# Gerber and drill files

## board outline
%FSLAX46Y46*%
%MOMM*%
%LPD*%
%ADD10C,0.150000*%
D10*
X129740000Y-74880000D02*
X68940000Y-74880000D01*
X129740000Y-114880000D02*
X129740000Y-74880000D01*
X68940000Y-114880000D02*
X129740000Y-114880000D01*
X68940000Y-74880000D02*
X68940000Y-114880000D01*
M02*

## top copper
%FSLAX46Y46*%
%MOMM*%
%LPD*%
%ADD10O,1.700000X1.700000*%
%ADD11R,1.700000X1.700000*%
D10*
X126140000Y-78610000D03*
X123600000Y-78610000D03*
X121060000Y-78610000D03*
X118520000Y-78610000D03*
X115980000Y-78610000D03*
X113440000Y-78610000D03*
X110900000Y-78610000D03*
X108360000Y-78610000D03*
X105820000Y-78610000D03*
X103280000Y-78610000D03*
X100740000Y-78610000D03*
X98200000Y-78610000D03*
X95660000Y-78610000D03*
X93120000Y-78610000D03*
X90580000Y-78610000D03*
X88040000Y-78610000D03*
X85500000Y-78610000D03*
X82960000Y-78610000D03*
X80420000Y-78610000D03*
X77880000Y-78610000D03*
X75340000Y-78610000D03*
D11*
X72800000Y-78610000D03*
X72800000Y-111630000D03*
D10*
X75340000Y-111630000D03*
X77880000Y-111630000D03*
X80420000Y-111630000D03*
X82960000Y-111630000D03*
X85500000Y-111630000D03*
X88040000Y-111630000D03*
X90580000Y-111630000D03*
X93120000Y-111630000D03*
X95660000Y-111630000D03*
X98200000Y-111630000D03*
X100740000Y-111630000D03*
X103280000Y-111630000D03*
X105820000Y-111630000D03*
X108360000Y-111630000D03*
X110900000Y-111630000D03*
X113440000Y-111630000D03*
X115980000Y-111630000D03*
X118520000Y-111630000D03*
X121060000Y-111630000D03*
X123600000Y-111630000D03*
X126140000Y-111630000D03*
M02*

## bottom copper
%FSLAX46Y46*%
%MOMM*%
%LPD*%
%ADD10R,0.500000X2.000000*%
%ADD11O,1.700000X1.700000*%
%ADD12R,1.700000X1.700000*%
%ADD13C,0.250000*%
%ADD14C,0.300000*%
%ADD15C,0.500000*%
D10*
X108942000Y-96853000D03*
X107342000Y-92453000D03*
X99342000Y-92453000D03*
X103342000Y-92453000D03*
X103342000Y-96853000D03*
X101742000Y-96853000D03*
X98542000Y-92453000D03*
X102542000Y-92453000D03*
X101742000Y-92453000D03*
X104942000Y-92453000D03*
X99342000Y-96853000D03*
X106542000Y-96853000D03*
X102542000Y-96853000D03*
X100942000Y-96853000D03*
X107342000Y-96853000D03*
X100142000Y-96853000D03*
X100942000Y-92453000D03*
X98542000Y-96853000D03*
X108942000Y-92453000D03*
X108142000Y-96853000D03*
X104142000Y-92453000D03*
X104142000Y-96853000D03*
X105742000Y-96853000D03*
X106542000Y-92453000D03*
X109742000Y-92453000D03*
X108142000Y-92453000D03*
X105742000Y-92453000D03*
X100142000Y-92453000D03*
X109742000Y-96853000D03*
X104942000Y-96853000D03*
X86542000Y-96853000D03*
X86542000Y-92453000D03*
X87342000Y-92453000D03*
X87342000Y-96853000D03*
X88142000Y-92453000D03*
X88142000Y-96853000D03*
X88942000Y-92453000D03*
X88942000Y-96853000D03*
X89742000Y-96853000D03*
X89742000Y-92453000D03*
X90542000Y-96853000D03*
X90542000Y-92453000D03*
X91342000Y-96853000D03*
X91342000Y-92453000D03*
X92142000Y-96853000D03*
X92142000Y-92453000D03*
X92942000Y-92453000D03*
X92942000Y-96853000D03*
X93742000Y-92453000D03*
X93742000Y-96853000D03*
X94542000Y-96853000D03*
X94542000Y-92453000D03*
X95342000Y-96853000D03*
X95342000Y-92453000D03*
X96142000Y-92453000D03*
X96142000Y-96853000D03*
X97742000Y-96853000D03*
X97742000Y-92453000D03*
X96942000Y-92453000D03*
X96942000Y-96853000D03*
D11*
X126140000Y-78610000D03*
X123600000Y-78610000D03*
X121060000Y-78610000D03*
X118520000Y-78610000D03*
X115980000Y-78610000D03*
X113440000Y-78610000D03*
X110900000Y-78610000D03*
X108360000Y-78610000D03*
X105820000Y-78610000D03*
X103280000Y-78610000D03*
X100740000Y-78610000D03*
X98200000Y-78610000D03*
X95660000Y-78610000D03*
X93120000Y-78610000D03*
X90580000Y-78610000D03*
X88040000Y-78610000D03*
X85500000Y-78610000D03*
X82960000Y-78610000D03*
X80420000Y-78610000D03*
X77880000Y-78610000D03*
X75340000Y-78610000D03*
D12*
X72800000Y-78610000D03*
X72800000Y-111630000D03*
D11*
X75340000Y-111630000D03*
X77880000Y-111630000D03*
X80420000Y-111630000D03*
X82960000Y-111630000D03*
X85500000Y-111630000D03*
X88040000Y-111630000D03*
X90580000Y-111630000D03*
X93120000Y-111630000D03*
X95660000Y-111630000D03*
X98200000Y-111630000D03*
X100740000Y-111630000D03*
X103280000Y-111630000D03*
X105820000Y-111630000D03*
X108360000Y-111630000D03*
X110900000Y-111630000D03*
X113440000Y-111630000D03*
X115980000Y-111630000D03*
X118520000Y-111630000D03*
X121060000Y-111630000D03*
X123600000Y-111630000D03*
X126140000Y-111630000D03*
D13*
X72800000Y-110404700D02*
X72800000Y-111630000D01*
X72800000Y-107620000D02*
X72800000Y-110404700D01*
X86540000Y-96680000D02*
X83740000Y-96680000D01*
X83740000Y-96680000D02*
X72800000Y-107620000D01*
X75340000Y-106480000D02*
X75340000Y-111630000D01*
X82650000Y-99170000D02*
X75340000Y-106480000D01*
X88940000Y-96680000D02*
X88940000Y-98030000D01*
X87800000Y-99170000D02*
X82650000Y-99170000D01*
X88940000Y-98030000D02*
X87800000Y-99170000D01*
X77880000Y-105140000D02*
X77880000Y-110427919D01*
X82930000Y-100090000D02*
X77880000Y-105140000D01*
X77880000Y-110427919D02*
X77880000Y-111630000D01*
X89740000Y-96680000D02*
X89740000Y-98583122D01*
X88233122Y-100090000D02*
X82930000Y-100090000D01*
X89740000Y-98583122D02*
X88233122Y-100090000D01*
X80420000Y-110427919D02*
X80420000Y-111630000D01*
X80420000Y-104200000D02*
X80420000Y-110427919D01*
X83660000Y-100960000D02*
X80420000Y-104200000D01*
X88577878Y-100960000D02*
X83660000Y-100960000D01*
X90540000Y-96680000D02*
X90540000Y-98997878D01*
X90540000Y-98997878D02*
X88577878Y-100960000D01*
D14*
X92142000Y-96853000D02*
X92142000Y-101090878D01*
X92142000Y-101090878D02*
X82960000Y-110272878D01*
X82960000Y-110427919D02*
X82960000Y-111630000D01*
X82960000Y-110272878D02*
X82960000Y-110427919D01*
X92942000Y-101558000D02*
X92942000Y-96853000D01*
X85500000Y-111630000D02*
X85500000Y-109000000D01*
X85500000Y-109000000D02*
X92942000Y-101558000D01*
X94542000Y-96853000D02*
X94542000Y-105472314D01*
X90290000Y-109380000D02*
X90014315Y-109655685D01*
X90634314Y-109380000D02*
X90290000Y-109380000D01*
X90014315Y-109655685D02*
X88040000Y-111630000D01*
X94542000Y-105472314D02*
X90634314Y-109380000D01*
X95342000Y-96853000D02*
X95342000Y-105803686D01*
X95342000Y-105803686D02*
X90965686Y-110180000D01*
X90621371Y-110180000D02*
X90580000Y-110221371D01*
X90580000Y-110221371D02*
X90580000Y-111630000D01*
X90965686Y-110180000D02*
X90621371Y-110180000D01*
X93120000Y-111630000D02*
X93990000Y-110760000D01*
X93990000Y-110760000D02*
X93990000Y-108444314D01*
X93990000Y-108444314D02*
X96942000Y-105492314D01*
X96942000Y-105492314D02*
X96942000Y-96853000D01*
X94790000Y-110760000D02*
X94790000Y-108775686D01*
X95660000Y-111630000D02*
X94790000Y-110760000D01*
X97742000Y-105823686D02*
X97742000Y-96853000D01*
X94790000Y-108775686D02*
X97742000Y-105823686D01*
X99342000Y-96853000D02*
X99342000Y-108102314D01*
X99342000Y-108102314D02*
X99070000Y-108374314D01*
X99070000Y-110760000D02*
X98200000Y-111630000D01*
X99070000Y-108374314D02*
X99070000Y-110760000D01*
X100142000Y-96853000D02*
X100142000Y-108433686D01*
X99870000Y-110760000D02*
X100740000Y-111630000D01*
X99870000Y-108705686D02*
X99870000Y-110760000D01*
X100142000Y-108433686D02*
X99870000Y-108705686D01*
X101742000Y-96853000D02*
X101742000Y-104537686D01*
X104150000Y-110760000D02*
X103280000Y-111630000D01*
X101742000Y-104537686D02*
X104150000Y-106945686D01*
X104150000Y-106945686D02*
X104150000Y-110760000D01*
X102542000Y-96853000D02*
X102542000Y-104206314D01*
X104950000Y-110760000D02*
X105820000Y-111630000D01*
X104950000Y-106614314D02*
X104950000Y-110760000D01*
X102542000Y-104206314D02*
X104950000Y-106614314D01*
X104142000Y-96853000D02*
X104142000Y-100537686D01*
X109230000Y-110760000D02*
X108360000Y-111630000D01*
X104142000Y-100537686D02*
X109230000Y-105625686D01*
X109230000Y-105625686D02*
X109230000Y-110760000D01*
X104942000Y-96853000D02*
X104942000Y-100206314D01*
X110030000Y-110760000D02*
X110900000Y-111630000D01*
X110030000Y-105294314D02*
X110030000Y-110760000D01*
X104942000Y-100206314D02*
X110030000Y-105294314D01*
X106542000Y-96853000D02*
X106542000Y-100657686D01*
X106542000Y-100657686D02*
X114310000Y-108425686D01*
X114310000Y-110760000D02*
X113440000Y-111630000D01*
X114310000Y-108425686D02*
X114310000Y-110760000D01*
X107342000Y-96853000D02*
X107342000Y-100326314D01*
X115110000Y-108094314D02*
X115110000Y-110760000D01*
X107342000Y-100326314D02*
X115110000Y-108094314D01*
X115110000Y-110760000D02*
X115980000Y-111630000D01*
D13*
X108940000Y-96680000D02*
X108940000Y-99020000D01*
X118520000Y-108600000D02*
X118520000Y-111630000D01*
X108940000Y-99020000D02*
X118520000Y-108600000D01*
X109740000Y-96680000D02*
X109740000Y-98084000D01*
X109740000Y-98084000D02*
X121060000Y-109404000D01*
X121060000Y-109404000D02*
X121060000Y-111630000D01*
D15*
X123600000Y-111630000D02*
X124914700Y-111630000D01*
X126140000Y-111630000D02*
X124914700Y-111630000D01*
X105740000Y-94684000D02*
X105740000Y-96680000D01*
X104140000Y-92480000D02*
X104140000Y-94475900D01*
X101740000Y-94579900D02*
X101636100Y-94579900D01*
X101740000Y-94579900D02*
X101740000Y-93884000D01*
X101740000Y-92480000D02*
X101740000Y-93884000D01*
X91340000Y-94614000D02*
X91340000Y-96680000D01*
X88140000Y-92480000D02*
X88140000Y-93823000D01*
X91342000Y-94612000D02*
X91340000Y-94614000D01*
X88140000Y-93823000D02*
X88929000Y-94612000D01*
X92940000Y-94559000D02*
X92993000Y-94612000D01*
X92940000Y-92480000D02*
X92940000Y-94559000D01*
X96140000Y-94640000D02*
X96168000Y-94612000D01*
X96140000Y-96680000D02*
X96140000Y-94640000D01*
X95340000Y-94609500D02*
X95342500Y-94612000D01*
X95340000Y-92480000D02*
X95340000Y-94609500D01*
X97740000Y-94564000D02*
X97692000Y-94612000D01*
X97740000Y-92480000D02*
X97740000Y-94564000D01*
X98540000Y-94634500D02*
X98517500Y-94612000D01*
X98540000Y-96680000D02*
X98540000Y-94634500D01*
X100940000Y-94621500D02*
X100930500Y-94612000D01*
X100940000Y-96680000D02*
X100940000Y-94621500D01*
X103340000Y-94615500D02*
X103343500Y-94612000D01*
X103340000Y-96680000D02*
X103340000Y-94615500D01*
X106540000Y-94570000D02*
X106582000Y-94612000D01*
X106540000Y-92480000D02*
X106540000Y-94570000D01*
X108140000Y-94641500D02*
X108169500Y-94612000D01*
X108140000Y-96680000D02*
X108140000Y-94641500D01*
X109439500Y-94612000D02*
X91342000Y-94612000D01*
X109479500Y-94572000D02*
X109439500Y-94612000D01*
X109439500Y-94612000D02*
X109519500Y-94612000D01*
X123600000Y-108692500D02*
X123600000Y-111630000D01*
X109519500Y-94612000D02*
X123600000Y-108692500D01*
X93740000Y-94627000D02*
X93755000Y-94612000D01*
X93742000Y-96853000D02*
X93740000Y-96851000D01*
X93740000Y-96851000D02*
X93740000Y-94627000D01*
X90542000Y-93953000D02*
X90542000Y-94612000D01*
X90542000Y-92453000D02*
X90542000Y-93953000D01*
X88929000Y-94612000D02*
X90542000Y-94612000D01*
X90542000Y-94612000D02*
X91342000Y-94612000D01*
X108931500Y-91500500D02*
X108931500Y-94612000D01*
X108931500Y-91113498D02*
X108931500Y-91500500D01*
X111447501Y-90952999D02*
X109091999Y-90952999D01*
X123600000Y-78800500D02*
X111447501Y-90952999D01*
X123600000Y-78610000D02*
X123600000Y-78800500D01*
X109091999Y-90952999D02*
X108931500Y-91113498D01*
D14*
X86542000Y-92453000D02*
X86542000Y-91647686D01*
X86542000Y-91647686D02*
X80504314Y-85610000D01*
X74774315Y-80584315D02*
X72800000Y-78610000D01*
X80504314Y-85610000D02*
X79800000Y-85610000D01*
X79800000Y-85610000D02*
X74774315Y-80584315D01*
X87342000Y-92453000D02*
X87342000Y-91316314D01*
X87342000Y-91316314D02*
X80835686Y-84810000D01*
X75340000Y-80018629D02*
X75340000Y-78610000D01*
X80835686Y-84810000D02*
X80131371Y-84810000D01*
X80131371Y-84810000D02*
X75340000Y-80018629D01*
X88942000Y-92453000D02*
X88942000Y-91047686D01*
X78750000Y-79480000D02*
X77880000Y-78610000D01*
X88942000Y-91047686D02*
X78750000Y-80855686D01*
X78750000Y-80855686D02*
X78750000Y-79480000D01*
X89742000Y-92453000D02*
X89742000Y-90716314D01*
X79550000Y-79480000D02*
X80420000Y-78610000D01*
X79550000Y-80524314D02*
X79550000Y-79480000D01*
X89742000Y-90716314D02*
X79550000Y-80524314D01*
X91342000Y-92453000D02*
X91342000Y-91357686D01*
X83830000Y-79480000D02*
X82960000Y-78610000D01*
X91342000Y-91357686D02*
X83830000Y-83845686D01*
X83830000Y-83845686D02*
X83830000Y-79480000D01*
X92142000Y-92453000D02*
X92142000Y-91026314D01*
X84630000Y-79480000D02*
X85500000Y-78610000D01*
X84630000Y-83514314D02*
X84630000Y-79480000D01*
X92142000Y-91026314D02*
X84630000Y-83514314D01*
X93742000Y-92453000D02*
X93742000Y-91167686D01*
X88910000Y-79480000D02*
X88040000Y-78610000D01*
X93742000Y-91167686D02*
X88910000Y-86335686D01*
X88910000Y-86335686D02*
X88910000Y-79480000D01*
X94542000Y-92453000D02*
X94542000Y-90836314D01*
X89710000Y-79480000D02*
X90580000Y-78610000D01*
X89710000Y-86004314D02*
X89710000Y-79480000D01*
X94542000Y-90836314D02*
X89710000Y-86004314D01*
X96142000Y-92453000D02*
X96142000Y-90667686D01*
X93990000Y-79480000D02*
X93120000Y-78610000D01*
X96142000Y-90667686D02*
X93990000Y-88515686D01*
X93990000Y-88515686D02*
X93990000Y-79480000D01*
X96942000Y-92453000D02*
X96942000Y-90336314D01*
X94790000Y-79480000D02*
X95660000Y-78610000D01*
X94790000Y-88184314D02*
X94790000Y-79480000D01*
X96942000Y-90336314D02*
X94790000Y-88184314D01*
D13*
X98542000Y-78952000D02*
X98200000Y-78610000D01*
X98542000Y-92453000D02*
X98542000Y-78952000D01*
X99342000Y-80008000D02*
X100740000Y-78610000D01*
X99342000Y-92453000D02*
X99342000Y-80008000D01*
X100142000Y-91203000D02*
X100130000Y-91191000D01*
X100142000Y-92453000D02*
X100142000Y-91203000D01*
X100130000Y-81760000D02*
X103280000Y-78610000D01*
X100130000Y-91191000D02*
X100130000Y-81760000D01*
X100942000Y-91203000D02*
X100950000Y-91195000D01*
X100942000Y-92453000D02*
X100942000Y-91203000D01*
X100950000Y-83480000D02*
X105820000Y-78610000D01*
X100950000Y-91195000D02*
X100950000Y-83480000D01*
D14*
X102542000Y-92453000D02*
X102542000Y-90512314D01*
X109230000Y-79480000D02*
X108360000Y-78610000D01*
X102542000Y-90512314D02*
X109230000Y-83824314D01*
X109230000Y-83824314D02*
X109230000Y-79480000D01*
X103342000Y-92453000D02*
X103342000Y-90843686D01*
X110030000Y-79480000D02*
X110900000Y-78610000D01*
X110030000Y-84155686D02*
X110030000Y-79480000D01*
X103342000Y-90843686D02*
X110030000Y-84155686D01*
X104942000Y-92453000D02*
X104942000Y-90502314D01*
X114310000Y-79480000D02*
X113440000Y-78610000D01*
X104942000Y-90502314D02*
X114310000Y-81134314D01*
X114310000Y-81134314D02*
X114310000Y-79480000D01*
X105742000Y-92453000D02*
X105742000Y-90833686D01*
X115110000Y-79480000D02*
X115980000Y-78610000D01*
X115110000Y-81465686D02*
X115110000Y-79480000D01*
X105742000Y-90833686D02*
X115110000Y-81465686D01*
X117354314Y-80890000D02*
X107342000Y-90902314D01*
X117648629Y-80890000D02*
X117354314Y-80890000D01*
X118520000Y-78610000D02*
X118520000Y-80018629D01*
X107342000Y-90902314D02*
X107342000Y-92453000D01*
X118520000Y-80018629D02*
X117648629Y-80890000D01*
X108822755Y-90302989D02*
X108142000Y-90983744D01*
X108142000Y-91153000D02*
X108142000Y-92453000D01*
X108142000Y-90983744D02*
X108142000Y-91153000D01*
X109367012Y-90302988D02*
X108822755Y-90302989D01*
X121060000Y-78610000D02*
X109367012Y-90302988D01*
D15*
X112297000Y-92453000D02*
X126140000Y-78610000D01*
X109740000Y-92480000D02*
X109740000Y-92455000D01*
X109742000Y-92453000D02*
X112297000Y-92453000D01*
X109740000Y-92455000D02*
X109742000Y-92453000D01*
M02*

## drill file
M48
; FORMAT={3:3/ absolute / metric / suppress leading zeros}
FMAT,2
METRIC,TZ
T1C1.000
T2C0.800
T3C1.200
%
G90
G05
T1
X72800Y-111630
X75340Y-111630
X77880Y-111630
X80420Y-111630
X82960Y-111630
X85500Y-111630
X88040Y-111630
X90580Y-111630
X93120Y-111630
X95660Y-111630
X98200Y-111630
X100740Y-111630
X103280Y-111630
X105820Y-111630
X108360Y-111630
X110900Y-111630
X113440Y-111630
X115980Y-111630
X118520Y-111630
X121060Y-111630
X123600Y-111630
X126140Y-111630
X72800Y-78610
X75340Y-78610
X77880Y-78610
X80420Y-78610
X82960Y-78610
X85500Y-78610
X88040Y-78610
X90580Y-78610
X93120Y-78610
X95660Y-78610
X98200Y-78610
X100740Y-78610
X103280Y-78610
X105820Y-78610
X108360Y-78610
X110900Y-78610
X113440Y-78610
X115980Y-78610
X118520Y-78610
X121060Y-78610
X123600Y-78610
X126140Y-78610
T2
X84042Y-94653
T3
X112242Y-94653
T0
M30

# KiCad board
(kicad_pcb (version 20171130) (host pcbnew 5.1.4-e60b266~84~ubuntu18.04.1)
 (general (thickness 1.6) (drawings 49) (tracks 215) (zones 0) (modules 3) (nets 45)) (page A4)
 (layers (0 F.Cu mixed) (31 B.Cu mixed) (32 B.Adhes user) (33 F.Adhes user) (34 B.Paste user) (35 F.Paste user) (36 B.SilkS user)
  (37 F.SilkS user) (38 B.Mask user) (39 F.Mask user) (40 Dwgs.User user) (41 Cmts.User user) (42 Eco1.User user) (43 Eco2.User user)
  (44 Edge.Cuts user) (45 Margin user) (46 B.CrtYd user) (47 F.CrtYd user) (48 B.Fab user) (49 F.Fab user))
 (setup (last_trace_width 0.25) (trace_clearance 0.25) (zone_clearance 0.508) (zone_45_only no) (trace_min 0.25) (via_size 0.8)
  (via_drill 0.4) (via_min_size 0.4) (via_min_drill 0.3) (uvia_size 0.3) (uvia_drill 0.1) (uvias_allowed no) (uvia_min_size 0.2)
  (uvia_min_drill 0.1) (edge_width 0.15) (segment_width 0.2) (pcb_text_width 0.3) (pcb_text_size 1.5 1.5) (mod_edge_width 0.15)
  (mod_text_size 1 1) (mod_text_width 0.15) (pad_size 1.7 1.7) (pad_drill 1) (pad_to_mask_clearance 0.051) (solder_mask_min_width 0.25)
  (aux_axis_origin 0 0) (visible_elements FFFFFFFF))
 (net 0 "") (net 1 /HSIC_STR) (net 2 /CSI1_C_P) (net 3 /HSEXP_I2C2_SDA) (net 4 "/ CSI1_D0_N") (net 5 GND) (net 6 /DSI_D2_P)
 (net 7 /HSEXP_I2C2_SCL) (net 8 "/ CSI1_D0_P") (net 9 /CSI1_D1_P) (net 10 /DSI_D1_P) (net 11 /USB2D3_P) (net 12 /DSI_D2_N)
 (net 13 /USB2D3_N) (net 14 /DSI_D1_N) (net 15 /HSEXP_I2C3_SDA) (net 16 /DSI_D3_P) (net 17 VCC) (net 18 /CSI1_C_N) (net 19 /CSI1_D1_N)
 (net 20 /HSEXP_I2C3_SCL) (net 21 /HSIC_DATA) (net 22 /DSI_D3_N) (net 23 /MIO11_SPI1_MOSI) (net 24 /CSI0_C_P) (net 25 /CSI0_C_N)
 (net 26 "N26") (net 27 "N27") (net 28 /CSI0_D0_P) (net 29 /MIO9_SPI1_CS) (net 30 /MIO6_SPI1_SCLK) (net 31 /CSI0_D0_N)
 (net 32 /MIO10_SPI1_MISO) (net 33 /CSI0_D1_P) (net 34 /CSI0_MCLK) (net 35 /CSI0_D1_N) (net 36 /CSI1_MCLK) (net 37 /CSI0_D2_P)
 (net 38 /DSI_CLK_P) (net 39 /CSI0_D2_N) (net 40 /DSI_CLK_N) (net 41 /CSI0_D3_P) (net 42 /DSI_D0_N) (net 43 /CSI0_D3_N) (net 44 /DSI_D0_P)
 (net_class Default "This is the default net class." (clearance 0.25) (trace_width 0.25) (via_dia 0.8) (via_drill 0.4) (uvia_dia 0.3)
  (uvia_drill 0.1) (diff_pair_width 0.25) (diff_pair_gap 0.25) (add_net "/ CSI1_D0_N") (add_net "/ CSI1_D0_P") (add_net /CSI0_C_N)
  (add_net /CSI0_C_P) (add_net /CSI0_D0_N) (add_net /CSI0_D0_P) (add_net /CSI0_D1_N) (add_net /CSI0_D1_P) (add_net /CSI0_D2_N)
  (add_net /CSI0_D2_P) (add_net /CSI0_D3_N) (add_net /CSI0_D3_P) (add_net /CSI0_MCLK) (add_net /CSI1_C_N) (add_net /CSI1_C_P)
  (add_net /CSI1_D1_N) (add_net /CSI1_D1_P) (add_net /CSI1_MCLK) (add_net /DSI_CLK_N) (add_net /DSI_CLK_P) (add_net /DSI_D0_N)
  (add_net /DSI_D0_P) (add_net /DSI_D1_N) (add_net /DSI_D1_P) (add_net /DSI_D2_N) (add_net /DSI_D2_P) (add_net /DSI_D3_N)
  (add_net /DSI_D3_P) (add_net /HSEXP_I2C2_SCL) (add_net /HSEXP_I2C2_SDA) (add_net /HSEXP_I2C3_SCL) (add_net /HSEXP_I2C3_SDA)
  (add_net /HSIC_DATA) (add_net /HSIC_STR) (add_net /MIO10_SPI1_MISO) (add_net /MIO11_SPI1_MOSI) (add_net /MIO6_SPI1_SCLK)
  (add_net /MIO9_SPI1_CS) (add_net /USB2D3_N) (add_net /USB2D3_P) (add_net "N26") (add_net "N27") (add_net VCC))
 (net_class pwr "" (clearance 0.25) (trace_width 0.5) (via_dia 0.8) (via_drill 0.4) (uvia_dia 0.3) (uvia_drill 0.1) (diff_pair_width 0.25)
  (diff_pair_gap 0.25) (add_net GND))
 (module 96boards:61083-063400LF (layer B.Cu) (at 98.142 94.653)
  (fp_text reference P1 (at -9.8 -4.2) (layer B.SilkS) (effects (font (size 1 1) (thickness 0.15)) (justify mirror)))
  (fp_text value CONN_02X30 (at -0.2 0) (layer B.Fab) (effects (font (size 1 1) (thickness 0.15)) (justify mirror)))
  (pad 57 smd rect (at 10.8 2.2) (size 0.5 2) (layers B.Cu B.Paste B.Mask) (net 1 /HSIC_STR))
  (pad 54 smd rect (at 9.2 -2.2) (size 0.5 2) (layers B.Cu B.Paste B.Mask) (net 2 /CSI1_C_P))
  (pad 34 smd rect (at 1.2 -2.2) (size 0.5 2) (layers B.Cu B.Paste B.Mask) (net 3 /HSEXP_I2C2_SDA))
  (pad 44 smd rect (at 5.2 -2.2) (size 0.5 2) (layers B.Cu B.Paste B.Mask) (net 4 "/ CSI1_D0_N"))
  (pad 43 smd rect (at 5.2 2.2) (size 0.5 2) (layers B.Cu B.Paste B.Mask) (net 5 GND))
  (pad 39 smd rect (at 3.6 2.2) (size 0.5 2) (layers B.Cu B.Paste B.Mask) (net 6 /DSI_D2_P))
  (pad 32 smd rect (at 0.4 -2.2) (size 0.5 2) (layers B.Cu B.Paste B.Mask) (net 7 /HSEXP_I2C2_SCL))
  (pad 42 smd rect (at 4.4 -2.2) (size 0.5 2) (layers B.Cu B.Paste B.Mask) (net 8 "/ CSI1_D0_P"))
  (pad 40 smd rect (at 3.6 -2.2) (size 0.5 2) (layers B.Cu B.Paste B.Mask) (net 5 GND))
  (pad 48 smd rect (at 6.8 -2.2) (size 0.5 2) (layers B.Cu B.Paste B.Mask) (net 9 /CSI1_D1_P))
  (pad 33 smd rect (at 1.2 2.2) (size 0.5 2) (layers B.Cu B.Paste B.Mask) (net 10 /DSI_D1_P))
  (pad 51 smd rect (at 8.4 2.2) (size 0.5 2) (layers B.Cu B.Paste B.Mask) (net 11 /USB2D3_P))
  (pad 41 smd rect (at 4.4 2.2) (size 0.5 2) (layers B.Cu B.Paste B.Mask) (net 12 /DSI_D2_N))
  (pad 37 smd rect (at 2.8 2.2) (size 0.5 2) (layers B.Cu B.Paste B.Mask) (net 5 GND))
  (pad 53 smd rect (at 9.2 2.2) (size 0.5 2) (layers B.Cu B.Paste B.Mask) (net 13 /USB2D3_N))
  (pad 35 smd rect (at 2 2.2) (size 0.5 2) (layers B.Cu B.Paste B.Mask) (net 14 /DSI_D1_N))
  (pad 38 smd rect (at 2.8 -2.2) (size 0.5 2) (layers B.Cu B.Paste B.Mask) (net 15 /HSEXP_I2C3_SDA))
  (pad 31 smd rect (at 0.4 2.2) (size 0.5 2) (layers B.Cu B.Paste B.Mask) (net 5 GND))
  (pad 58 smd rect (at 10.8 -2.2) (size 0.5 2) (layers B.Cu B.Paste B.Mask) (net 5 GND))
  (pad 55 smd rect (at 10 2.2) (size 0.5 2) (layers B.Cu B.Paste B.Mask) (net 5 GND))
  (pad 46 smd rect (at 6 -2.2) (size 0.5 2) (layers B.Cu B.Paste B.Mask) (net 5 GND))
  (pad 45 smd rect (at 6 2.2) (size 0.5 2) (layers B.Cu B.Paste B.Mask) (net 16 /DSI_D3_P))
  (pad 49 smd rect (at 7.6 2.2) (size 0.5 2) (layers B.Cu B.Paste B.Mask) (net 5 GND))
  (pad 52 smd rect (at 8.4 -2.2) (size 0.5 2) (layers B.Cu B.Paste B.Mask) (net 5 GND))
  (pad 60 smd rect (at 11.6 -2.2) (size 0.5 2) (layers B.Cu B.Paste B.Mask) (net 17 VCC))
  (pad 56 smd rect (at 10 -2.2) (size 0.5 2) (layers B.Cu B.Paste B.Mask) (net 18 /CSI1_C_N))
  (pad 50 smd rect (at 7.6 -2.2) (size 0.5 2) (layers B.Cu B.Paste B.Mask) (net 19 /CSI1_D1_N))
  (pad 36 smd rect (at 2 -2.2) (size 0.5 2) (layers B.Cu B.Paste B.Mask) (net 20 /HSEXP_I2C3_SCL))
  (pad 59 smd rect (at 11.6 2.2) (size 0.5 2) (layers B.Cu B.Paste B.Mask) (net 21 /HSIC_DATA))
  (pad 47 smd rect (at 6.8 2.2) (size 0.5 2) (layers B.Cu B.Paste B.Mask) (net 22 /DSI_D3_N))
  (pad "" np_thru_hole circle (at 14.1 0) (size 1.2 1.2) (drill 1.2) (layers *.Cu *.Mask))
  (pad 1 smd rect (at -11.6 2.2) (size 0.5 2) (layers B.Cu B.Paste B.Mask) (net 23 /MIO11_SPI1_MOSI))
  (pad 2 smd rect (at -11.6 -2.2) (size 0.5 2) (layers B.Cu B.Paste B.Mask) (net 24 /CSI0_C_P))
  (pad 4 smd rect (at -10.8 -2.2) (size 0.5 2) (layers B.Cu B.Paste B.Mask) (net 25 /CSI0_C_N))
  (pad 3 smd rect (at -10.8 2.2) (size 0.5 2) (layers B.Cu B.Paste B.Mask) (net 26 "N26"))
  (pad 6 smd rect (at -10 -2.2) (size 0.5 2) (layers B.Cu B.Paste B.Mask) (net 5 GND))
  (pad 5 smd rect (at -10 2.2) (size 0.5 2) (layers B.Cu B.Paste B.Mask) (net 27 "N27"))
  (pad 8 smd rect (at -9.2 -2.2) (size 0.5 2) (layers B.Cu B.Paste B.Mask) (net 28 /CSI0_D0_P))
  (pad 7 smd rect (at -9.2 2.2) (size 0.5 2) (layers B.Cu B.Paste B.Mask) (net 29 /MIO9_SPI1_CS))
  (pad 9 smd rect (at -8.4 2.2) (size 0.5 2) (layers B.Cu B.Paste B.Mask) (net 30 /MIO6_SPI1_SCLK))
  (pad 10 smd rect (at -8.4 -2.2) (size 0.5 2) (layers B.Cu B.Paste B.Mask) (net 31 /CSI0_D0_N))
  (pad 11 smd rect (at -7.6 2.2) (size 0.5 2) (layers B.Cu B.Paste B.Mask) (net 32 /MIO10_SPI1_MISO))
  (pad 12 smd rect (at -7.6 -2.2) (size 0.5 2) (layers B.Cu B.Paste B.Mask) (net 5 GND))
  (pad 13 smd rect (at -6.8 2.2) (size 0.5 2) (layers B.Cu B.Paste B.Mask) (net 5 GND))
  (pad 14 smd rect (at -6.8 -2.2) (size 0.5 2) (layers B.Cu B.Paste B.Mask) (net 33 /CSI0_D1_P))
  (pad 15 smd rect (at -6 2.2) (size 0.5 2) (layers B.Cu B.Paste B.Mask) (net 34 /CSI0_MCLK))
  (pad 16 smd rect (at -6 -2.2) (size 0.5 2) (layers B.Cu B.Paste B.Mask) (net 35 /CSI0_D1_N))
  (pad 18 smd rect (at -5.2 -2.2) (size 0.5 2) (layers B.Cu B.Paste B.Mask) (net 5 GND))
  (pad 17 smd rect (at -5.2 2.2) (size 0.5 2) (layers B.Cu B.Paste B.Mask) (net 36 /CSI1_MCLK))
  (pad 20 smd rect (at -4.4 -2.2) (size 0.5 2) (layers B.Cu B.Paste B.Mask) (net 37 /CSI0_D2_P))
  (pad 19 smd rect (at -4.4 2.2) (size 0.5 2) (layers B.Cu B.Paste B.Mask) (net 5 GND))
  (pad 21 smd rect (at -3.6 2.2) (size 0.5 2) (layers B.Cu B.Paste B.Mask) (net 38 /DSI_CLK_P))
  (pad 22 smd rect (at -3.6 -2.2) (size 0.5 2) (layers B.Cu B.Paste B.Mask) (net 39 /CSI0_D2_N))
  (pad 23 smd rect (at -2.8 2.2) (size 0.5 2) (layers B.Cu B.Paste B.Mask) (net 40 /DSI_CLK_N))
  (pad 24 smd rect (at -2.8 -2.2) (size 0.5 2) (layers B.Cu B.Paste B.Mask) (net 5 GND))
  (pad 26 smd rect (at -2 -2.2) (size 0.5 2) (layers B.Cu B.Paste B.Mask) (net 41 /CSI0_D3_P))
  (pad 25 smd rect (at -2 2.2) (size 0.5 2) (layers B.Cu B.Paste B.Mask) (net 5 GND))
  (pad 29 smd rect (at -0.4 2.2) (size 0.5 2) (layers B.Cu B.Paste B.Mask) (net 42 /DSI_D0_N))
  (pad 30 smd rect (at -0.4 -2.2) (size 0.5 2) (layers B.Cu B.Paste B.Mask) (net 5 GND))
  (pad 28 smd rect (at -1.2 -2.2) (size 0.5 2) (layers B.Cu B.Paste B.Mask) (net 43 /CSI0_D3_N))
  (pad 27 smd rect (at -1.2 2.2) (size 0.5 2) (layers B.Cu B.Paste B.Mask) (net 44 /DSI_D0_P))
  (pad "" np_thru_hole circle (at -14.1 0) (size 0.8 0.8) (drill 0.8) (layers *.Cu *.Mask)))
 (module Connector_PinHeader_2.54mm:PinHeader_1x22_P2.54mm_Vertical (layer F.Cu) (at 72.8 78.61 90)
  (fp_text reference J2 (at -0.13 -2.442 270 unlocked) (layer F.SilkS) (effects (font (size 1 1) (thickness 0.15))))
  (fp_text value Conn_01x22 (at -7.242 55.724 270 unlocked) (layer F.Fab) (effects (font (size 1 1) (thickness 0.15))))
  (pad 22 thru_hole oval (at 0 53.34 90) (size 1.7 1.7) (drill 1) (layers *.Cu *.Mask) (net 17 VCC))
  (pad 21 thru_hole oval (at 0 50.8 90) (size 1.7 1.7) (drill 1) (layers *.Cu *.Mask) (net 5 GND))
  (pad 20 thru_hole oval (at 0 48.26 90) (size 1.7 1.7) (drill 1) (layers *.Cu *.Mask) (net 18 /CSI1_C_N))
  (pad 19 thru_hole oval (at 0 45.72 90) (size 1.7 1.7) (drill 1) (layers *.Cu *.Mask) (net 2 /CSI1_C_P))
  (pad 18 thru_hole oval (at 0 43.18 90) (size 1.7 1.7) (drill 1) (layers *.Cu *.Mask) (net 19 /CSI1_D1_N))
  (pad 17 thru_hole oval (at 0 40.64 90) (size 1.7 1.7) (drill 1) (layers *.Cu *.Mask) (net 9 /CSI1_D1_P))
  (pad 16 thru_hole oval (at 0 38.1 90) (size 1.7 1.7) (drill 1) (layers *.Cu *.Mask) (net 4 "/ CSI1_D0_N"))
  (pad 15 thru_hole oval (at 0 35.56 90) (size 1.7 1.7) (drill 1) (layers *.Cu *.Mask) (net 8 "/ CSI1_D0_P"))
  (pad 14 thru_hole oval (at 0 33.02 90) (size 1.7 1.7) (drill 1) (layers *.Cu *.Mask) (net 15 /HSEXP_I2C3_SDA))
  (pad 13 thru_hole oval (at 0 30.48 90) (size 1.7 1.7) (drill 1) (layers *.Cu *.Mask) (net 20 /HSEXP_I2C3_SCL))
  (pad 12 thru_hole oval (at 0 27.94 90) (size 1.7 1.7) (drill 1) (layers *.Cu *.Mask) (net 3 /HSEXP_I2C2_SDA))
  (pad 11 thru_hole oval (at 0 25.4 90) (size 1.7 1.7) (drill 1) (layers *.Cu *.Mask) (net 7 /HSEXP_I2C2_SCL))
  (pad 10 thru_hole oval (at 0 22.86 90) (size 1.7 1.7) (drill 1) (layers *.Cu *.Mask) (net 43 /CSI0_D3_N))
  (pad 9 thru_hole oval (at 0 20.32 90) (size 1.7 1.7) (drill 1) (layers *.Cu *.Mask) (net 41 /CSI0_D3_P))
  (pad 8 thru_hole oval (at 0 17.78 90) (size 1.7 1.7) (drill 1) (layers *.Cu *.Mask) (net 39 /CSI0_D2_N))
  (pad 7 thru_hole oval (at 0 15.24 90) (size 1.7 1.7) (drill 1) (layers *.Cu *.Mask) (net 37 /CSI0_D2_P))
  (pad 6 thru_hole oval (at 0 12.7 90) (size 1.7 1.7) (drill 1) (layers *.Cu *.Mask) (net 35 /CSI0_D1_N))
  (pad 5 thru_hole oval (at 0 10.16 90) (size 1.7 1.7) (drill 1) (layers *.Cu *.Mask) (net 33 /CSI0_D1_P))
  (pad 4 thru_hole oval (at 0 7.62 90) (size 1.7 1.7) (drill 1) (layers *.Cu *.Mask) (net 31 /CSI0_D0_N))
  (pad 3 thru_hole oval (at 0 5.08 90) (size 1.7 1.7) (drill 1) (layers *.Cu *.Mask) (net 28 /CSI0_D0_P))
  (pad 2 thru_hole oval (at 0 2.54 90) (size 1.7 1.7) (drill 1) (layers *.Cu *.Mask) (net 25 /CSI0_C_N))
  (pad 1 thru_hole rect (at 0 0 90) (size 1.7 1.7) (drill 1) (layers *.Cu *.Mask) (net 24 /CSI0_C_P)))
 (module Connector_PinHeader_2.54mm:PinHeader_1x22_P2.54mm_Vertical (layer F.Cu) (at 72.8 111.63 90)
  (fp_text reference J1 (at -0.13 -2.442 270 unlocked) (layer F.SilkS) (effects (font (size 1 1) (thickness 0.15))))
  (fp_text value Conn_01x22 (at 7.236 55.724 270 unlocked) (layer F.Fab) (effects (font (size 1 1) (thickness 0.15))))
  (pad 1 thru_hole rect (at 0 0 90) (size 1.7 1.7) (drill 1) (layers *.Cu *.SilkS *.Mask) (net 23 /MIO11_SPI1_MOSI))
  (pad 2 thru_hole oval (at 0 2.54 90) (size 1.7 1.7) (drill 1) (layers *.Cu *.Mask) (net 29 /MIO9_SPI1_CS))
  (pad 3 thru_hole oval (at 0 5.08 90) (size 1.7 1.7) (drill 1) (layers *.Cu *.Mask) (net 30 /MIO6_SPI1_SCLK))
  (pad 4 thru_hole oval (at 0 7.62 90) (size 1.7 1.7) (drill 1) (layers *.Cu *.Mask) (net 32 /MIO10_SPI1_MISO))
  (pad 5 thru_hole oval (at 0 10.16 90) (size 1.7 1.7) (drill 1) (layers *.Cu *.Mask) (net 34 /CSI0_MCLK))
  (pad 6 thru_hole oval (at 0 12.7 90) (size 1.7 1.7) (drill 1) (layers *.Cu *.Mask) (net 36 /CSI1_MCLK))
  (pad 7 thru_hole oval (at 0 15.24 90) (size 1.7 1.7) (drill 1) (layers *.Cu *.Mask) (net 38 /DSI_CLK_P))
  (pad 8 thru_hole oval (at 0 17.78 90) (size 1.7 1.7) (drill 1) (layers *.Cu *.Mask) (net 40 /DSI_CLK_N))
  (pad 9 thru_hole oval (at 0 20.32 90) (size 1.7 1.7) (drill 1) (layers *.Cu *.Mask) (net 44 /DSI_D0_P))
  (pad 10 thru_hole oval (at 0 22.86 90) (size 1.7 1.7) (drill 1) (layers *.Cu *.Mask) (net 42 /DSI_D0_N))
  (pad 11 thru_hole oval (at 0 25.4 90) (size 1.7 1.7) (drill 1) (layers *.Cu *.Mask) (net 10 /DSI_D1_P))
  (pad 12 thru_hole oval (at 0 27.94 90) (size 1.7 1.7) (drill 1) (layers *.Cu *.Mask) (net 14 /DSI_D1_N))
  (pad 13 thru_hole oval (at 0 30.48 90) (size 1.7 1.7) (drill 1) (layers *.Cu *.Mask) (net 6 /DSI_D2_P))
  (pad 14 thru_hole oval (at 0 33.02 90) (size 1.7 1.7) (drill 1) (layers *.Cu *.Mask) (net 12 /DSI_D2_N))
  (pad 15 thru_hole oval (at 0 35.56 90) (size 1.7 1.7) (drill 1) (layers *.Cu *.Mask) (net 16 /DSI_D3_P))
  (pad 16 thru_hole oval (at 0 38.1 90) (size 1.7 1.7) (drill 1) (layers *.Cu *.Mask) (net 22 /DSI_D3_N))
  (pad 17 thru_hole oval (at 0 40.64 90) (size 1.7 1.7) (drill 1) (layers *.Cu *.Mask) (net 11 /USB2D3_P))
  (pad 18 thru_hole oval (at 0 43.18 90) (size 1.7 1.7) (drill 1) (layers *.Cu *.Mask) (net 13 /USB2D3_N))
  (pad 19 thru_hole oval (at 0 45.72 90) (size 1.7 1.7) (drill 1) (layers *.Cu *.Mask) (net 1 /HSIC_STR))
  (pad 20 thru_hole oval (at 0 48.26 90) (size 1.7 1.7) (drill 1) (layers *.Cu *.Mask) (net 21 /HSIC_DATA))
  (pad 21 thru_hole oval (at 0 50.8 90) (size 1.7 1.7) (drill 1) (layers *.Cu *.Mask) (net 5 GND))
  (pad 22 thru_hole oval (at 0 53.34 90) (size 1.7 1.7) (drill 1) (layers *.Cu *.Mask) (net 5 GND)))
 (gr_line (start 129.74 74.88) (end 68.94 74.88) (layer Edge.Cuts) (width 0.15))
 (gr_line (start 129.74 114.88) (end 129.74 74.88) (layer Edge.Cuts) (width 0.15))
 (gr_line (start 68.94 114.88) (end 129.74 114.88) (layer Edge.Cuts) (width 0.15))
 (gr_line (start 68.94 74.88) (end 68.94 114.88) (layer Edge.Cuts) (width 0.15))
 (segment (start 72.8 110.4047) (end 72.8 111.63) (width 0.25) (layer B.Cu) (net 23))
 (segment (start 72.8 107.62) (end 72.8 110.4047) (width 0.25) (layer B.Cu) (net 23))
 (segment (start 86.54 96.68) (end 83.74 96.68) (width 0.25) (layer B.Cu) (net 23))
 (segment (start 83.74 96.68) (end 72.8 107.62) (width 0.25) (layer B.Cu) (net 23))
 (segment (start 75.34 106.48) (end 75.34 111.63) (width 0.25) (layer B.Cu) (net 29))
 (segment (start 82.65 99.17) (end 75.34 106.48) (width 0.25) (layer B.Cu) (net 29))
 (segment (start 88.94 96.68) (end 88.94 98.03) (width 0.25) (layer B.Cu) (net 29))
 (segment (start 87.8 99.17) (end 82.65 99.17) (width 0.25) (layer B.Cu) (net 29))
 (segment (start 88.94 98.03) (end 87.8 99.17) (width 0.25) (layer B.Cu) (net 29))
 (segment (start 77.88 105.14) (end 77.88 110.427919) (width 0.25) (layer B.Cu) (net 30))
 (segment (start 82.93 100.09) (end 77.88 105.14) (width 0.25) (layer B.Cu) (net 30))
 (segment (start 77.88 110.427919) (end 77.88 111.63) (width 0.25) (layer B.Cu) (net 30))
 (segment (start 89.74 96.68) (end 89.74 98.583122) (width 0.25) (layer B.Cu) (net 30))
 (segment (start 88.233122 100.09) (end 82.93 100.09) (width 0.25) (layer B.Cu) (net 30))
 (segment (start 89.74 98.583122) (end 88.233122 100.09) (width 0.25) (layer B.Cu) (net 30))
 (segment (start 80.42 110.427919) (end 80.42 111.63) (width 0.25) (layer B.Cu) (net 32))
 (segment (start 80.42 104.2) (end 80.42 110.427919) (width 0.25) (layer B.Cu) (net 32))
 (segment (start 83.66 100.96) (end 80.42 104.2) (width 0.25) (layer B.Cu) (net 32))
 (segment (start 88.577878 100.96) (end 83.66 100.96) (width 0.25) (layer B.Cu) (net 32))
 (segment (start 90.54 96.68) (end 90.54 98.997878) (width 0.25) (layer B.Cu) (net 32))
 (segment (start 90.54 98.997878) (end 88.577878 100.96) (width 0.25) (layer B.Cu) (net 32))
 (segment (start 92.142 96.853) (end 92.142 101.090878) (width 0.3) (layer B.Cu) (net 34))
 (segment (start 92.142 101.090878) (end 82.96 110.272878) (width 0.3) (layer B.Cu) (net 34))
 (segment (start 82.96 110.427919) (end 82.96 111.63) (width 0.3) (layer B.Cu) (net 34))
 (segment (start 82.96 110.272878) (end 82.96 110.427919) (width 0.3) (layer B.Cu) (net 34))
 (segment (start 92.942 101.558) (end 92.942 96.853) (width 0.3) (layer B.Cu) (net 36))
 (segment (start 85.5 111.63) (end 85.5 109) (width 0.3) (layer B.Cu) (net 36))
 (segment (start 85.5 109) (end 92.942 101.558) (width 0.3) (layer B.Cu) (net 36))
 (segment (start 94.542 96.853) (end 94.542 105.472314) (width 0.3) (layer B.Cu) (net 38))
 (segment (start 90.29 109.38) (end 90.014315 109.655685) (width 0.3) (layer B.Cu) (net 38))
 (segment (start 90.634314 109.38) (end 90.29 109.38) (width 0.3) (layer B.Cu) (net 38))
 (segment (start 90.014315 109.655685) (end 88.04 111.63) (width 0.3) (layer B.Cu) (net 38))
 (segment (start 94.542 105.472314) (end 90.634314 109.38) (width 0.3) (layer B.Cu) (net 38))
 (segment (start 95.342 96.853) (end 95.342 105.803686) (width 0.3) (layer B.Cu) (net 40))
 (segment (start 95.342 105.803686) (end 90.965686 110.18) (width 0.3) (layer B.Cu) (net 40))
 (segment (start 90.621371 110.18) (end 90.58 110.221371) (width 0.3) (layer B.Cu) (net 40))
 (segment (start 90.58 110.221371) (end 90.58 111.63) (width 0.3) (layer B.Cu) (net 40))
 (segment (start 90.965686 110.18) (end 90.621371 110.18) (width 0.3) (layer B.Cu) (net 40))
 (segment (start 93.12 111.63) (end 93.99 110.76) (width 0.3) (layer B.Cu) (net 44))
 (segment (start 93.99 110.76) (end 93.99 108.444314) (width 0.3) (layer B.Cu) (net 44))
 (segment (start 93.99 108.444314) (end 96.942 105.492314) (width 0.3) (layer B.Cu) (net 44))
 (segment (start 96.942 105.492314) (end 96.942 96.853) (width 0.3) (layer B.Cu) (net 44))
 (segment (start 94.79 110.76) (end 94.79 108.775686) (width 0.3) (layer B.Cu) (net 42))
 (segment (start 95.66 111.63) (end 94.79 110.76) (width 0.3) (layer B.Cu) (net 42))
 (segment (start 97.742 105.823686) (end 97.742 96.853) (width 0.3) (layer B.Cu) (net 42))
 (segment (start 94.79 108.775686) (end 97.742 105.823686) (width 0.3) (layer B.Cu) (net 42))
 (segment (start 99.342 96.853) (end 99.342 108.102314) (width 0.3) (layer B.Cu) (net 10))
 (segment (start 99.342 108.102314) (end 99.07 108.374314) (width 0.3) (layer B.Cu) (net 10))
 (segment (start 99.07 110.76) (end 98.2 111.63) (width 0.3) (layer B.Cu) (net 10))
 (segment (start 99.07 108.374314) (end 99.07 110.76) (width 0.3) (layer B.Cu) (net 10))
 (segment (start 100.142 96.853) (end 100.142 108.433686) (width 0.3) (layer B.Cu) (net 14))
 (segment (start 99.87 110.76) (end 100.74 111.63) (width 0.3) (layer B.Cu) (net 14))
 (segment (start 99.87 108.705686) (end 99.87 110.76) (width 0.3) (layer B.Cu) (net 14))
 (segment (start 100.142 108.433686) (end 99.87 108.705686) (width 0.3) (layer B.Cu) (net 14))
 (segment (start 101.742 96.853) (end 101.742 104.537686) (width 0.3) (layer B.Cu) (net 6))
 (segment (start 104.15 110.76) (end 103.28 111.63) (width 0.3) (layer B.Cu) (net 6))
 (segment (start 101.742 104.537686) (end 104.15 106.945686) (width 0.3) (layer B.Cu) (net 6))
 (segment (start 104.15 106.945686) (end 104.15 110.76) (width 0.3) (layer B.Cu) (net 6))
 (segment (start 102.542 96.853) (end 102.542 104.206314) (width 0.3) (layer B.Cu) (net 12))
 (segment (start 104.95 110.76) (end 105.82 111.63) (width 0.3) (layer B.Cu) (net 12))
 (segment (start 104.95 106.614314) (end 104.95 110.76) (width 0.3) (layer B.Cu) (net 12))
 (segment (start 102.542 104.206314) (end 104.95 106.614314) (width 0.3) (layer B.Cu) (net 12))
 (segment (start 104.142 96.853) (end 104.142 100.537686) (width 0.3) (layer B.Cu) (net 16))
 (segment (start 109.23 110.76) (end 108.36 111.63) (width 0.3) (layer B.Cu) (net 16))
 (segment (start 104.142 100.537686) (end 109.23 105.625686) (width 0.3) (layer B.Cu) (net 16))
 (segment (start 109.23 105.625686) (end 109.23 110.76) (width 0.3) (layer B.Cu) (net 16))
 (segment (start 104.942 96.853) (end 104.942 100.206314) (width 0.3) (layer B.Cu) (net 22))
 (segment (start 110.03 110.76) (end 110.9 111.63) (width 0.3) (layer B.Cu) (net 22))
 (segment (start 110.03 105.294314) (end 110.03 110.76) (width 0.3) (layer B.Cu) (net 22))
 (segment (start 104.942 100.206314) (end 110.03 105.294314) (width 0.3) (layer B.Cu) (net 22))
 (segment (start 106.542 96.853) (end 106.542 100.657686) (width 0.3) (layer B.Cu) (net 11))
 (segment (start 106.542 100.657686) (end 114.31 108.425686) (width 0.3) (layer B.Cu) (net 11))
 (segment (start 114.31 110.76) (end 113.44 111.63) (width 0.3) (layer B.Cu) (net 11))
 (segment (start 114.31 108.425686) (end 114.31 110.76) (width 0.3) (layer B.Cu) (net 11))
 (segment (start 107.342 96.853) (end 107.342 100.326314) (width 0.3) (layer B.Cu) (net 13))
 (segment (start 115.11 108.094314) (end 115.11 110.76) (width 0.3) (layer B.Cu) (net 13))
 (segment (start 107.342 100.326314) (end 115.11 108.094314) (width 0.3) (layer B.Cu) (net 13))
 (segment (start 115.11 110.76) (end 115.98 111.63) (width 0.3) (layer B.Cu) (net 13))
 (segment (start 108.94 96.68) (end 108.94 99.02) (width 0.25) (layer B.Cu) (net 1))
 (segment (start 118.52 108.6) (end 118.52 111.63) (width 0.25) (layer B.Cu) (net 1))
 (segment (start 108.94 99.02) (end 118.52 108.6) (width 0.25) (layer B.Cu) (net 1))
 (segment (start 109.74 96.68) (end 109.74 98.084) (width 0.25) (layer B.Cu) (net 21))
 (segment (start 109.74 98.084) (end 121.06 109.404) (width 0.25) (layer B.Cu) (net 21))
 (segment (start 121.06 109.404) (end 121.06 111.63) (width 0.25) (layer B.Cu) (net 21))
 (segment (start 123.6 111.63) (end 124.9147 111.63) (width 0.5) (layer B.Cu) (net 5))
 (segment (start 126.14 111.63) (end 124.9147 111.63) (width 0.5) (layer B.Cu) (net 5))
 (segment (start 105.74 94.684) (end 105.74 96.68) (width 0.5) (layer B.Cu) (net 5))
 (segment (start 104.14 92.48) (end 104.14 94.4759) (width 0.5) (layer B.Cu) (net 5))
 (segment (start 101.74 94.5799) (end 101.6361 94.5799) (width 0.5) (layer B.Cu) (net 5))
 (segment (start 101.74 94.5799) (end 101.74 93.884) (width 0.5) (layer B.Cu) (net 5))
 (segment (start 101.74 92.48) (end 101.74 93.884) (width 0.5) (layer B.Cu) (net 5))
 (segment (start 91.34 94.614) (end 91.34 96.68) (width 0.5) (layer B.Cu) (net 5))
 (segment (start 88.14 92.48) (end 88.14 93.823) (width 0.5) (layer B.Cu) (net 5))
 (segment (start 91.342 94.612) (end 91.34 94.614) (width 0.5) (layer B.Cu) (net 5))
 (segment (start 88.14 93.823) (end 88.929 94.612) (width 0.5) (layer B.Cu) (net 5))
 (segment (start 92.94 94.559) (end 92.993 94.612) (width 0.5) (layer B.Cu) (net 5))
 (segment (start 92.94 92.48) (end 92.94 94.559) (width 0.5) (layer B.Cu) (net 5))
 (segment (start 96.14 94.64) (end 96.168 94.612) (width 0.5) (layer B.Cu) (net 5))
 (segment (start 96.14 96.68) (end 96.14 94.64) (width 0.5) (layer B.Cu) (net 5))
 (segment (start 95.34 94.6095) (end 95.3425 94.612) (width 0.5) (layer B.Cu) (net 5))
 (segment (start 95.34 92.48) (end 95.34 94.6095) (width 0.5) (layer B.Cu) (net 5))
 (segment (start 97.74 94.564) (end 97.692 94.612) (width 0.5) (layer B.Cu) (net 5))
 (segment (start 97.74 92.48) (end 97.74 94.564) (width 0.5) (layer B.Cu) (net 5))
 (segment (start 98.54 94.6345) (end 98.5175 94.612) (width 0.5) (layer B.Cu) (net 5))
 (segment (start 98.54 96.68) (end 98.54 94.6345) (width 0.5) (layer B.Cu) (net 5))
 (segment (start 100.94 94.6215) (end 100.9305 94.612) (width 0.5) (layer B.Cu) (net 5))
 (segment (start 100.94 96.68) (end 100.94 94.6215) (width 0.5) (layer B.Cu) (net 5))
 (segment (start 103.34 94.6155) (end 103.3435 94.612) (width 0.5) (layer B.Cu) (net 5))
 (segment (start 103.34 96.68) (end 103.34 94.6155) (width 0.5) (layer B.Cu) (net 5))
 (segment (start 106.54 94.57) (end 106.582 94.612) (width 0.5) (layer B.Cu) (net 5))
 (segment (start 106.54 92.48) (end 106.54 94.57) (width 0.5) (layer B.Cu) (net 5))
 (segment (start 108.14 94.6415) (end 108.1695 94.612) (width 0.5) (layer B.Cu) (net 5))
 (segment (start 108.14 96.68) (end 108.14 94.6415) (width 0.5) (layer B.Cu) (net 5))
 (segment (start 109.4395 94.612) (end 91.342 94.612) (width 0.5) (layer B.Cu) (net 5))
 (segment (start 109.4795 94.572) (end 109.4395 94.612) (width 0.5) (layer B.Cu) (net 5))
 (segment (start 109.4395 94.612) (end 109.5195 94.612) (width 0.5) (layer B.Cu) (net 5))
 (segment (start 123.6 108.6925) (end 123.6 111.63) (width 0.5) (layer B.Cu) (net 5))
 (segment (start 109.5195 94.612) (end 123.6 108.6925) (width 0.5) (layer B.Cu) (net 5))
 (segment (start 93.74 94.627) (end 93.755 94.612) (width 0.5) (layer B.Cu) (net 5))
 (segment (start 93.742 96.853) (end 93.74 96.851) (width 0.5) (layer B.Cu) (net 5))
 (segment (start 93.74 96.851) (end 93.74 94.627) (width 0.5) (layer B.Cu) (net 5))
 (segment (start 90.542 93.953) (end 90.542 94.612) (width 0.5) (layer B.Cu) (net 5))
 (segment (start 90.542 92.453) (end 90.542 93.953) (width 0.5) (layer B.Cu) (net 5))
 (segment (start 88.929 94.612) (end 90.542 94.612) (width 0.5) (layer B.Cu) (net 5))
 (segment (start 90.542 94.612) (end 91.342 94.612) (width 0.5) (layer B.Cu) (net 5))
 (segment (start 108.9315 91.5005) (end 108.9315 94.612) (width 0.5) (layer B.Cu) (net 5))
 (segment (start 108.9315 91.113498) (end 108.9315 91.5005) (width 0.5) (layer B.Cu) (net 5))
 (segment (start 111.447501 90.952999) (end 109.091999 90.952999) (width 0.5) (layer B.Cu) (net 5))
 (segment (start 123.6 78.8005) (end 111.447501 90.952999) (width 0.5) (layer B.Cu) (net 5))
 (segment (start 123.6 78.61) (end 123.6 78.8005) (width 0.5) (layer B.Cu) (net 5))
 (segment (start 109.091999 90.952999) (end 108.9315 91.113498) (width 0.5) (layer B.Cu) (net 5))
 (segment (start 86.542 92.453) (end 86.542 91.647686) (width 0.3) (layer B.Cu) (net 24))
 (segment (start 86.542 91.647686) (end 80.504314 85.61) (width 0.3) (layer B.Cu) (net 24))
 (segment (start 74.774315 80.584315) (end 72.8 78.61) (width 0.3) (layer B.Cu) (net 24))
 (segment (start 80.504314 85.61) (end 79.8 85.61) (width 0.3) (layer B.Cu) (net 24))
 (segment (start 79.8 85.61) (end 74.774315 80.584315) (width 0.3) (layer B.Cu) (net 24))
 (segment (start 87.342 92.453) (end 87.342 91.316314) (width 0.3) (layer B.Cu) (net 25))
 (segment (start 87.342 91.316314) (end 80.835686 84.81) (width 0.3) (layer B.Cu) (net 25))
 (segment (start 75.34 80.018629) (end 75.34 78.61) (width 0.3) (layer B.Cu) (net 25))
 (segment (start 80.835686 84.81) (end 80.131371 84.81) (width 0.3) (layer B.Cu) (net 25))
 (segment (start 80.131371 84.81) (end 75.34 80.018629) (width 0.3) (layer B.Cu) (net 25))
 (segment (start 88.942 92.453) (end 88.942 91.047686) (width 0.3) (layer B.Cu) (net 28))
 (segment (start 78.75 79.48) (end 77.88 78.61) (width 0.3) (layer B.Cu) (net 28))
 (segment (start 88.942 91.047686) (end 78.75 80.855686) (width 0.3) (layer B.Cu) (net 28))
 (segment (start 78.75 80.855686) (end 78.75 79.48) (width 0.3) (layer B.Cu) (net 28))
 (segment (start 89.742 92.453) (end 89.742 90.716314) (width 0.3) (layer B.Cu) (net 31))
 (segment (start 79.55 79.48) (end 80.42 78.61) (width 0.3) (layer B.Cu) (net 31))
 (segment (start 79.55 80.524314) (end 79.55 79.48) (width 0.3) (layer B.Cu) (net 31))
 (segment (start 89.742 90.716314) (end 79.55 80.524314) (width 0.3) (layer B.Cu) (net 31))
 (segment (start 91.342 92.453) (end 91.342 91.357686) (width 0.3) (layer B.Cu) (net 33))
 (segment (start 83.83 79.48) (end 82.96 78.61) (width 0.3) (layer B.Cu) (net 33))
 (segment (start 91.342 91.357686) (end 83.83 83.845686) (width 0.3) (layer B.Cu) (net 33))
 (segment (start 83.83 83.845686) (end 83.83 79.48) (width 0.3) (layer B.Cu) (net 33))
 (segment (start 92.142 92.453) (end 92.142 91.026314) (width 0.3) (layer B.Cu) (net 35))
 (segment (start 84.63 79.48) (end 85.5 78.61) (width 0.3) (layer B.Cu) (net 35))
 (segment (start 84.63 83.514314) (end 84.63 79.48) (width 0.3) (layer B.Cu) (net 35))
 (segment (start 92.142 91.026314) (end 84.63 83.514314) (width 0.3) (layer B.Cu) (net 35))
 (segment (start 93.742 92.453) (end 93.742 91.167686) (width 0.3) (layer B.Cu) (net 37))
 (segment (start 88.91 79.48) (end 88.04 78.61) (width 0.3) (layer B.Cu) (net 37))
 (segment (start 93.742 91.167686) (end 88.91 86.335686) (width 0.3) (layer B.Cu) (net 37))
 (segment (start 88.91 86.335686) (end 88.91 79.48) (width 0.3) (layer B.Cu) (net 37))
 (segment (start 94.542 92.453) (end 94.542 90.836314) (width 0.3) (layer B.Cu) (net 39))
 (segment (start 89.71 79.48) (end 90.58 78.61) (width 0.3) (layer B.Cu) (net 39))
 (segment (start 89.71 86.004314) (end 89.71 79.48) (width 0.3) (layer B.Cu) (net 39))
 (segment (start 94.542 90.836314) (end 89.71 86.004314) (width 0.3) (layer B.Cu) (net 39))
 (segment (start 96.142 92.453) (end 96.142 90.667686) (width 0.3) (layer B.Cu) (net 41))
 (segment (start 93.99 79.48) (end 93.12 78.61) (width 0.3) (layer B.Cu) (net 41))
 (segment (start 96.142 90.667686) (end 93.99 88.515686) (width 0.3) (layer B.Cu) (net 41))
 (segment (start 93.99 88.515686) (end 93.99 79.48) (width 0.3) (layer B.Cu) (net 41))
 (segment (start 96.942 92.453) (end 96.942 90.336314) (width 0.3) (layer B.Cu) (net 43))
 (segment (start 94.79 79.48) (end 95.66 78.61) (width 0.3) (layer B.Cu) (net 43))
 (segment (start 94.79 88.184314) (end 94.79 79.48) (width 0.3) (layer B.Cu) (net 43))
 (segment (start 96.942 90.336314) (end 94.79 88.184314) (width 0.3) (layer B.Cu) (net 43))
 (segment (start 98.542 78.952) (end 98.2 78.61) (width 0.25) (layer B.Cu) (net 7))
 (segment (start 98.542 92.453) (end 98.542 78.952) (width 0.25) (layer B.Cu) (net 7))
 (segment (start 99.342 80.008) (end 100.74 78.61) (width 0.25) (layer B.Cu) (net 3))
 (segment (start 99.342 92.453) (end 99.342 80.008) (width 0.25) (layer B.Cu) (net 3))
 (segment (start 100.142 91.203) (end 100.13 91.191) (width 0.25) (layer B.Cu) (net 20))
 (segment (start 100.142 92.453) (end 100.142 91.203) (width 0.25) (layer B.Cu) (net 20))
 (segment (start 100.13 81.76) (end 103.28 78.61) (width 0.25) (layer B.Cu) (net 20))
 (segment (start 100.13 91.191) (end 100.13 81.76) (width 0.25) (layer B.Cu) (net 20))
 (segment (start 100.942 91.203) (end 100.95 91.195) (width 0.25) (layer B.Cu) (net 15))
 (segment (start 100.942 92.453) (end 100.942 91.203) (width 0.25) (layer B.Cu) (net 15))
 (segment (start 100.95 83.48) (end 105.82 78.61) (width 0.25) (layer B.Cu) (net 15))
 (segment (start 100.95 91.195) (end 100.95 83.48) (width 0.25) (layer B.Cu) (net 15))
 (segment (start 102.542 92.453) (end 102.542 90.512314) (width 0.3) (layer B.Cu) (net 8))
 (segment (start 109.23 79.48) (end 108.36 78.61) (width 0.3) (layer B.Cu) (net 8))
 (segment (start 102.542 90.512314) (end 109.23 83.824314) (width 0.3) (layer B.Cu) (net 8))
 (segment (start 109.23 83.824314) (end 109.23 79.48) (width 0.3) (layer B.Cu) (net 8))
 (segment (start 103.342 92.453) (end 103.342 90.843686) (width 0.3) (layer B.Cu) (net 4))
 (segment (start 110.03 79.48) (end 110.9 78.61) (width 0.3) (layer B.Cu) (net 4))
 (segment (start 110.03 84.155686) (end 110.03 79.48) (width 0.3) (layer B.Cu) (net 4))
 (segment (start 103.342 90.843686) (end 110.03 84.155686) (width 0.3) (layer B.Cu) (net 4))
 (segment (start 104.942 92.453) (end 104.942 90.502314) (width 0.3) (layer B.Cu) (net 9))
 (segment (start 114.31 79.48) (end 113.44 78.61) (width 0.3) (layer B.Cu) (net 9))
 (segment (start 104.942 90.502314) (end 114.31 81.134314) (width 0.3) (layer B.Cu) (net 9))
 (segment (start 114.31 81.134314) (end 114.31 79.48) (width 0.3) (layer B.Cu) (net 9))
 (segment (start 105.742 92.453) (end 105.742 90.833686) (width 0.3) (layer B.Cu) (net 19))
 (segment (start 115.11 79.48) (end 115.98 78.61) (width 0.3) (layer B.Cu) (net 19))
 (segment (start 115.11 81.465686) (end 115.11 79.48) (width 0.3) (layer B.Cu) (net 19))
 (segment (start 105.742 90.833686) (end 115.11 81.465686) (width 0.3) (layer B.Cu) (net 19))
 (segment (start 117.354314 80.89) (end 107.342 90.902314) (width 0.3) (layer B.Cu) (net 2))
 (segment (start 117.648629 80.89) (end 117.354314 80.89) (width 0.3) (layer B.Cu) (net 2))
 (segment (start 118.52 78.61) (end 118.52 80.018629) (width 0.3) (layer B.Cu) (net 2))
 (segment (start 107.342 90.902314) (end 107.342 92.453) (width 0.3) (layer B.Cu) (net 2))
 (segment (start 118.52 80.018629) (end 117.648629 80.89) (width 0.3) (layer B.Cu) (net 2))
 (segment (start 108.822755 90.302989) (end 108.142 90.983744) (width 0.3) (layer B.Cu) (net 18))
 (segment (start 108.142 91.153) (end 108.142 92.453) (width 0.3) (layer B.Cu) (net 18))
 (segment (start 108.142 90.983744) (end 108.142 91.153) (width 0.3) (layer B.Cu) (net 18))
 (segment (start 109.367012 90.302988) (end 108.822755 90.302989) (width 0.3) (layer B.Cu) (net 18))
 (segment (start 121.06 78.61) (end 109.367012 90.302988) (width 0.3) (layer B.Cu) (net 18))
 (segment (start 112.297 92.453) (end 126.14 78.61) (width 0.5) (layer B.Cu) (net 17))
 (segment (start 109.74 92.48) (end 109.74 92.455) (width 0.5) (layer B.Cu) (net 17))
 (segment (start 109.742 92.453) (end 112.297 92.453) (width 0.5) (layer B.Cu) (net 17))
 (segment (start 109.74 92.455) (end 109.742 92.453) (width 0.5) (layer B.Cu) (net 17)))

